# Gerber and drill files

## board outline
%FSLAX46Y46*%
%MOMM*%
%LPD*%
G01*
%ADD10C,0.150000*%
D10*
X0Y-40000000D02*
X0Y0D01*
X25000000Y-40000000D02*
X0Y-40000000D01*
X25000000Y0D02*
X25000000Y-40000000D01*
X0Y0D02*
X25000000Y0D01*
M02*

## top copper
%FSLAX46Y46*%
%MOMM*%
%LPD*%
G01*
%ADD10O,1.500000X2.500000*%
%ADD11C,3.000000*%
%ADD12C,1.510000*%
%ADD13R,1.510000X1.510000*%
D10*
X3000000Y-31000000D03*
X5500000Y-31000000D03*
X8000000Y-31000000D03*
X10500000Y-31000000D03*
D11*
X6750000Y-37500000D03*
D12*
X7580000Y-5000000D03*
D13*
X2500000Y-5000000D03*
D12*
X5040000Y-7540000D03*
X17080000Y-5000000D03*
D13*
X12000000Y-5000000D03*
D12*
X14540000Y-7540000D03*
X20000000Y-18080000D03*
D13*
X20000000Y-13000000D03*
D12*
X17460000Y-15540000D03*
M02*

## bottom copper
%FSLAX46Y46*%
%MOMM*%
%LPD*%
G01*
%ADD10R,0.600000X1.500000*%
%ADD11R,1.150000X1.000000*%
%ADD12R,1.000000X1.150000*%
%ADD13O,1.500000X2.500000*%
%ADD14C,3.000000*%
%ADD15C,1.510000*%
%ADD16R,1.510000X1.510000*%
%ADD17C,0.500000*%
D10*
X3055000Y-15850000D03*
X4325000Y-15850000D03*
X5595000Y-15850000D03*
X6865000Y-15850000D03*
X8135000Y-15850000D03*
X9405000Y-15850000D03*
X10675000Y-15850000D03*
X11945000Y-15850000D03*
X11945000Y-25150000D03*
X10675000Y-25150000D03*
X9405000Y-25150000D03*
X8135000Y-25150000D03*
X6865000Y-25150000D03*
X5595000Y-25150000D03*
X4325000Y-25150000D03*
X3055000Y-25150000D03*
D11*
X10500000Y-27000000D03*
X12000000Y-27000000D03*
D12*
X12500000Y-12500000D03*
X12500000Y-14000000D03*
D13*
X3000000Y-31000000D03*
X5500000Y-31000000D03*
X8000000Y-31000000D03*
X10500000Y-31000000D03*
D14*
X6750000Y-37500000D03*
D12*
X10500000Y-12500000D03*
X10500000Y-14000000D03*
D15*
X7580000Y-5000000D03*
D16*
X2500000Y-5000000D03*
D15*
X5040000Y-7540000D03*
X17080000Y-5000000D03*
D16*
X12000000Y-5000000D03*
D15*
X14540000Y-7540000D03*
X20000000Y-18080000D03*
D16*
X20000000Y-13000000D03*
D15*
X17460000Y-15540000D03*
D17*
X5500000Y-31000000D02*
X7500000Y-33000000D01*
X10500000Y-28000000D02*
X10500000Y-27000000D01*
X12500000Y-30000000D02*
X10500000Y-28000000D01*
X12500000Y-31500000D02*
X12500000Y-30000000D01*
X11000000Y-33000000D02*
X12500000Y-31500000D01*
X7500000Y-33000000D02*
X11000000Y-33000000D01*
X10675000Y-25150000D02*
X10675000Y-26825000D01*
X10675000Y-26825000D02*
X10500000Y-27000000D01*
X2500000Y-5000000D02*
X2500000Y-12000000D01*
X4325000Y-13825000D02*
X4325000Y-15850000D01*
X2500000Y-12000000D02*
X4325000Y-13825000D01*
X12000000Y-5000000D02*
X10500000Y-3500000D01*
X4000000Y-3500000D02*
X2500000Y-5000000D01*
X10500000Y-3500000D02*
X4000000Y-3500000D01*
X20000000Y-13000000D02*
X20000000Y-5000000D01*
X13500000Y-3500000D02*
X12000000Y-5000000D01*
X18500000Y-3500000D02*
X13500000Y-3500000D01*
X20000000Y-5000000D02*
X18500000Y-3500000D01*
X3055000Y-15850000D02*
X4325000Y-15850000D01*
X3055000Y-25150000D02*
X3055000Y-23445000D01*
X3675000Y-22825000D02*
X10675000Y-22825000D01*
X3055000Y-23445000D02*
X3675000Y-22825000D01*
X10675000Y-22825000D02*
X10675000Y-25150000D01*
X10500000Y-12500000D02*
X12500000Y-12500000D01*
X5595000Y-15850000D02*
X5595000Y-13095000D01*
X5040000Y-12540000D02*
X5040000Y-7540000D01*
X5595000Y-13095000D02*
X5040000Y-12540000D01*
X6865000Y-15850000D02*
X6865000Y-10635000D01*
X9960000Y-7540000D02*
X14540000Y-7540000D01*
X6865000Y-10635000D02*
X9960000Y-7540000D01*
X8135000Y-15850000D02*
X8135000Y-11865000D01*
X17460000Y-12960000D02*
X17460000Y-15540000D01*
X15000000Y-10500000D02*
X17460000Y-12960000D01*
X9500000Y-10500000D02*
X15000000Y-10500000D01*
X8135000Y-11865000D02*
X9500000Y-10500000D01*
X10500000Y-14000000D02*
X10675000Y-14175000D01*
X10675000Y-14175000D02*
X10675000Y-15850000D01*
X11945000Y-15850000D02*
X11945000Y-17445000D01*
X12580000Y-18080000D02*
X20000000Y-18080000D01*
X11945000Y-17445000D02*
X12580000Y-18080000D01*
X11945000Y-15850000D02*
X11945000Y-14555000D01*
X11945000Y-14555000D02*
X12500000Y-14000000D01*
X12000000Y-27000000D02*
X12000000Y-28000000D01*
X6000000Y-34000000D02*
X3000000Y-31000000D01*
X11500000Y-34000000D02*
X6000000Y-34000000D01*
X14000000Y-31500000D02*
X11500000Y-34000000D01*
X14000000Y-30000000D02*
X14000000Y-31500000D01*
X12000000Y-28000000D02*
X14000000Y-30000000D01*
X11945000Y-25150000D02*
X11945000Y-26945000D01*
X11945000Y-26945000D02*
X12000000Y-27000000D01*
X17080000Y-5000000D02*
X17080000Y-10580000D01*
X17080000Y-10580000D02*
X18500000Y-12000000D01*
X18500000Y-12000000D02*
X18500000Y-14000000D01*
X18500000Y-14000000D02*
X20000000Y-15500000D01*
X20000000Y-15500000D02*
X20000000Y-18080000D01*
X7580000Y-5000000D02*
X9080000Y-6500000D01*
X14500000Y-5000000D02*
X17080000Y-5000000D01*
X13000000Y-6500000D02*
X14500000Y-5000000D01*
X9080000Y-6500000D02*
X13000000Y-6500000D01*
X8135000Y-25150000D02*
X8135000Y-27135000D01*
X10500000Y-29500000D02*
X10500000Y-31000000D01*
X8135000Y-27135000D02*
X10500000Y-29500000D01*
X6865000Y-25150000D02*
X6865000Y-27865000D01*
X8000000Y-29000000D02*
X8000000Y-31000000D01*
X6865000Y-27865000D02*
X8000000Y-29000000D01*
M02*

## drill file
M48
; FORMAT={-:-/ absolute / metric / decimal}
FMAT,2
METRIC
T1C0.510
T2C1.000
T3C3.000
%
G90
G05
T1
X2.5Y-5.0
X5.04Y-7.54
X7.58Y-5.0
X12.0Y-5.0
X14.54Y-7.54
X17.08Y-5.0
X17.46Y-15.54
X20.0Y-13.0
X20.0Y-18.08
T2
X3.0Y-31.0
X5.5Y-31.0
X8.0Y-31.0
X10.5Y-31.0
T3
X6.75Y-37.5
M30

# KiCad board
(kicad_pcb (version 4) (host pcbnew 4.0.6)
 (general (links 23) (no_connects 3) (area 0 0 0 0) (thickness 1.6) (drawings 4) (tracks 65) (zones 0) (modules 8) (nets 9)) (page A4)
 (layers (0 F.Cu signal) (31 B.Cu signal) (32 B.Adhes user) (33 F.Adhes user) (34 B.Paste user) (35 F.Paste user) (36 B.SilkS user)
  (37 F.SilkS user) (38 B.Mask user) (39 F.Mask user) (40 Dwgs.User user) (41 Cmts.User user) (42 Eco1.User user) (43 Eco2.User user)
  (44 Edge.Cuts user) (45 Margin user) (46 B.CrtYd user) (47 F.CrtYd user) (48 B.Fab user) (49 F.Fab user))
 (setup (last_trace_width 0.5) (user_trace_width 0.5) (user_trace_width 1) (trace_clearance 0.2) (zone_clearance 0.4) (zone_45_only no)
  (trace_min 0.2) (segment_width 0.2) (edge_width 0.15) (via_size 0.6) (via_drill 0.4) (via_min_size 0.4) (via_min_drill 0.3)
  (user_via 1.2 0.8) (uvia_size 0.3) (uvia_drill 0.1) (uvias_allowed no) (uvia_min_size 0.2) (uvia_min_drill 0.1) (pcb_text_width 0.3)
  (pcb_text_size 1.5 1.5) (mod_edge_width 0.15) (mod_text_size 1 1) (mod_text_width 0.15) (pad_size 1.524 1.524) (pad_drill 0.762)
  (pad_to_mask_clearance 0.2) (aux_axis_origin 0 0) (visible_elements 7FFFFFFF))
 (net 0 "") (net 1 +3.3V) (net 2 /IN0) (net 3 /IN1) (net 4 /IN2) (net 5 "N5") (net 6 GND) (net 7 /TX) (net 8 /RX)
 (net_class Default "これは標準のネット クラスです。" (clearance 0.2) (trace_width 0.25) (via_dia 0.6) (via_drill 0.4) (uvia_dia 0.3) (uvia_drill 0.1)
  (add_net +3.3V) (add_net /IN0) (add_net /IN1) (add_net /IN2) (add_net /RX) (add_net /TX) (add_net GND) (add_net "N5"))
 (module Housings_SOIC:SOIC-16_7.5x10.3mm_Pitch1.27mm (layer B.Cu) (at 7.5 20.5 270)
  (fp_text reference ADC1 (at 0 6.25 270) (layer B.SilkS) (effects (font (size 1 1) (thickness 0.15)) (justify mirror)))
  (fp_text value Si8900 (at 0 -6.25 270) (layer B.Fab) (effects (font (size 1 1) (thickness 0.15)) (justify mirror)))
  (pad 1 smd rect (at -4.65 4.445 270) (size 1.5 0.6) (layers B.Cu B.Paste B.Mask) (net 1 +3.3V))
  (pad 2 smd rect (at -4.65 3.175 270) (size 1.5 0.6) (layers B.Cu B.Paste B.Mask) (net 1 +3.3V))
  (pad 3 smd rect (at -4.65 1.905 270) (size 1.5 0.6) (layers B.Cu B.Paste B.Mask) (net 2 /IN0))
  (pad 4 smd rect (at -4.65 0.635 270) (size 1.5 0.6) (layers B.Cu B.Paste B.Mask) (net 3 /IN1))
  (pad 5 smd rect (at -4.65 -0.635 270) (size 1.5 0.6) (layers B.Cu B.Paste B.Mask) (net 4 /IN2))
  (pad 6 smd rect (at -4.65 -1.905 270) (size 1.5 0.6) (layers B.Cu B.Paste B.Mask))
  (pad 7 smd rect (at -4.65 -3.175 270) (size 1.5 0.6) (layers B.Cu B.Paste B.Mask) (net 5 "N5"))
  (pad 8 smd rect (at -4.65 -4.445 270) (size 1.5 0.6) (layers B.Cu B.Paste B.Mask) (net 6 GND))
  (pad 9 smd rect (at 4.65 -4.445 270) (size 1.5 0.6) (layers B.Cu B.Paste B.Mask) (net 6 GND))
  (pad 10 smd rect (at 4.65 -3.175 270) (size 1.5 0.6) (layers B.Cu B.Paste B.Mask) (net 1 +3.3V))
  (pad 11 smd rect (at 4.65 -1.905 270) (size 1.5 0.6) (layers B.Cu B.Paste B.Mask))
  (pad 12 smd rect (at 4.65 -0.635 270) (size 1.5 0.6) (layers B.Cu B.Paste B.Mask) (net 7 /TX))
  (pad 13 smd rect (at 4.65 0.635 270) (size 1.5 0.6) (layers B.Cu B.Paste B.Mask) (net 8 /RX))
  (pad 14 smd rect (at 4.65 1.905 270) (size 1.5 0.6) (layers B.Cu B.Paste B.Mask))
  (pad 15 smd rect (at 4.65 3.175 270) (size 1.5 0.6) (layers B.Cu B.Paste B.Mask))
  (pad 16 smd rect (at 4.65 4.445 270) (size 1.5 0.6) (layers B.Cu B.Paste B.Mask) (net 1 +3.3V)))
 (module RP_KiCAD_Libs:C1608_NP (layer B.Cu) (at 11.5 27)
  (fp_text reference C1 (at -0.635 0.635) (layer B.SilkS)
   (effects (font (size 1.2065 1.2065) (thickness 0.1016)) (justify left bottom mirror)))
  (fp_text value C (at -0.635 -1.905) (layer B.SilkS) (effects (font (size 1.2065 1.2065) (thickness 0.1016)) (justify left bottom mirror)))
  (pad 1 smd rect (at -1 0) (size 1.15 1) (layers B.Cu B.Paste B.Mask) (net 1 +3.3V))
  (pad 2 smd rect (at 0.5 0) (size 1.15 1) (layers B.Cu B.Paste B.Mask) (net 6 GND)))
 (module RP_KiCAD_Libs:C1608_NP (layer B.Cu) (at 12.5 13.5 270)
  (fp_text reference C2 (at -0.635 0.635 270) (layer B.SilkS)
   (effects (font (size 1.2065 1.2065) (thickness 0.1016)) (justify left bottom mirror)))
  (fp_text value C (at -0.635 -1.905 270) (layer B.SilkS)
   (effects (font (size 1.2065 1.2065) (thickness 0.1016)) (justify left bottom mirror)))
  (pad 1 smd rect (at -1 0 270) (size 1.15 1) (layers B.Cu B.Paste B.Mask) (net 1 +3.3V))
  (pad 2 smd rect (at 0.5 0 270) (size 1.15 1) (layers B.Cu B.Paste B.Mask) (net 6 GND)))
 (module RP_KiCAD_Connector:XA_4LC (layer F.Cu) (at 3 31)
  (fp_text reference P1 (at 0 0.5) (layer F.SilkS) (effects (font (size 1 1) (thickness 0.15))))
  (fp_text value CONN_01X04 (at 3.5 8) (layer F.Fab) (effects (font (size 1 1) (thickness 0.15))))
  (pad 1 thru_hole oval (at 0 0) (size 1.5 2.5) (drill 1) (layers *.Cu *.Mask F.SilkS) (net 6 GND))
  (pad 2 thru_hole oval (at 2.5 0) (size 1.5 2.5) (drill 1) (layers *.Cu *.Mask F.SilkS) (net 1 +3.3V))
  (pad 3 thru_hole oval (at 5 0) (size 1.5 2.5) (drill 1) (layers *.Cu *.Mask F.SilkS) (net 8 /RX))
  (pad 4 thru_hole oval (at 7.5 0) (size 1.5 2.5) (drill 1) (layers *.Cu *.Mask F.SilkS) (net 7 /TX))
  (pad "" thru_hole circle (at 3.75 6.5) (size 3 3) (drill 3) (layers *.Cu *.Mask F.SilkS) (clearance -0.3)))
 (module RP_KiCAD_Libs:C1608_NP (layer B.Cu) (at 10.5 13.5 270)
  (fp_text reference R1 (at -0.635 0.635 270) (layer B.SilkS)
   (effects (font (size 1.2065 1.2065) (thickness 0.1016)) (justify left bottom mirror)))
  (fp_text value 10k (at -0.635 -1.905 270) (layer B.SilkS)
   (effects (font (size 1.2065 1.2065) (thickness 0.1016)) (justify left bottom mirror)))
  (pad 1 smd rect (at -1 0 270) (size 1.15 1) (layers B.Cu B.Paste B.Mask) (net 1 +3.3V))
  (pad 2 smd rect (at 0.5 0 270) (size 1.15 1) (layers B.Cu B.Paste B.Mask) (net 5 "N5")))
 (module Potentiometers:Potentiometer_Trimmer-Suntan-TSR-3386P (layer F.Cu) (at 2.5 5)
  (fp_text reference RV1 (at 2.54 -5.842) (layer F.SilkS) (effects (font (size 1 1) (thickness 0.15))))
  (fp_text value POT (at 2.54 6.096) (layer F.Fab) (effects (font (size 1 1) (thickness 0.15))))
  (pad 3 thru_hole circle (at 5.08 0) (size 1.51 1.51) (drill 0.51) (layers *.Cu *.Mask F.SilkS) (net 6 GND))
  (pad 1 thru_hole rect (at 0 0) (size 1.51 1.51) (drill 0.51) (layers *.Cu *.Mask F.SilkS) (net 1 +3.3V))
  (pad 2 thru_hole circle (at 2.54 2.54) (size 1.51 1.51) (drill 0.51) (layers *.Cu *.Mask F.SilkS) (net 2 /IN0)))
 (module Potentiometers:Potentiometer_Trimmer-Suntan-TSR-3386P (layer F.Cu) (at 12 5)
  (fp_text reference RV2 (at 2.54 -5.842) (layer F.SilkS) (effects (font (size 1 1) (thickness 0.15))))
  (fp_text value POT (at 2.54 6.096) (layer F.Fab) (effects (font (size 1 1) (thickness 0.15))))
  (pad 3 thru_hole circle (at 5.08 0) (size 1.51 1.51) (drill 0.51) (layers *.Cu *.Mask F.SilkS) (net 6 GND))
  (pad 1 thru_hole rect (at 0 0) (size 1.51 1.51) (drill 0.51) (layers *.Cu *.Mask F.SilkS) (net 1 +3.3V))
  (pad 2 thru_hole circle (at 2.54 2.54) (size 1.51 1.51) (drill 0.51) (layers *.Cu *.Mask F.SilkS) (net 3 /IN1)))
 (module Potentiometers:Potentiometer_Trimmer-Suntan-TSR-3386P (layer F.Cu) (at 20 13 270)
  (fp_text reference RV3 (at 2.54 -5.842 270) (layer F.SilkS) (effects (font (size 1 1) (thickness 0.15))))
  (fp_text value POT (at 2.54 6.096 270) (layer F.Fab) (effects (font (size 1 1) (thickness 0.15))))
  (pad 3 thru_hole circle (at 5.08 0 270) (size 1.51 1.51) (drill 0.51) (layers *.Cu *.Mask F.SilkS) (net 6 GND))
  (pad 1 thru_hole rect (at 0 0 270) (size 1.51 1.51) (drill 0.51) (layers *.Cu *.Mask F.SilkS) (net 1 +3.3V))
  (pad 2 thru_hole circle (at 2.54 2.54 270) (size 1.51 1.51) (drill 0.51) (layers *.Cu *.Mask F.SilkS) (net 4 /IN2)))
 (gr_line (start 0 40) (end 0 0) (angle 90) (layer Edge.Cuts) (width 0.15))
 (gr_line (start 25 40) (end 0 40) (angle 90) (layer Edge.Cuts) (width 0.15))
 (gr_line (start 25 0) (end 25 40) (angle 90) (layer Edge.Cuts) (width 0.15))
 (gr_line (start 0 0) (end 25 0) (angle 90) (layer Edge.Cuts) (width 0.15))
 (segment (start 5.5 31) (end 7.5 33) (width 0.5) (layer B.Cu) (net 1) (status 400000))
 (segment (start 10.5 28) (end 10.5 27) (width 0.5) (layer B.Cu) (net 1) (status 800000))
 (segment (start 12.5 30) (end 10.5 28) (width 0.5) (layer B.Cu) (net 1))
 (segment (start 12.5 31.5) (end 12.5 30) (width 0.5) (layer B.Cu) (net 1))
 (segment (start 11 33) (end 12.5 31.5) (width 0.5) (layer B.Cu) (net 1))
 (segment (start 7.5 33) (end 11 33) (width 0.5) (layer B.Cu) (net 1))
 (segment (start 10.675 25.15) (end 10.675 26.825) (width 0.5) (layer B.Cu) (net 1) (status C00000))
 (segment (start 10.675 26.825) (end 10.5 27) (width 0.5) (layer B.Cu) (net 1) (status C00000))
 (segment (start 2.5 5) (end 2.5 12) (width 0.5) (layer B.Cu) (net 1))
 (segment (start 4.325 13.825) (end 4.325 15.85) (width 0.5) (layer B.Cu) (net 1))
 (segment (start 2.5 12) (end 4.325 13.825) (width 0.5) (layer B.Cu) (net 1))
 (segment (start 12 5) (end 10.5 3.5) (width 0.5) (layer B.Cu) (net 1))
 (segment (start 4 3.5) (end 2.5 5) (width 0.5) (layer B.Cu) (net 1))
 (segment (start 10.5 3.5) (end 4 3.5) (width 0.5) (layer B.Cu) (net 1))
 (segment (start 20 13) (end 20 5) (width 0.5) (layer B.Cu) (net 1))
 (segment (start 13.5 3.5) (end 12 5) (width 0.5) (layer B.Cu) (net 1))
 (segment (start 18.5 3.5) (end 13.5 3.5) (width 0.5) (layer B.Cu) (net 1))
 (segment (start 20 5) (end 18.5 3.5) (width 0.5) (layer B.Cu) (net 1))
 (segment (start 3.055 15.85) (end 4.325 15.85) (width 0.5) (layer B.Cu) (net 1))
 (segment (start 3.055 25.15) (end 3.055 23.445) (width 0.5) (layer B.Cu) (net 1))
 (segment (start 3.675 22.825) (end 10.675 22.825) (width 0.5) (layer B.Cu) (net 1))
 (segment (start 3.055 23.445) (end 3.675 22.825) (width 0.5) (layer B.Cu) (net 1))
 (segment (start 10.675 22.825) (end 10.675 25.15) (width 0.5) (layer B.Cu) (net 1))
 (segment (start 10.5 12.5) (end 12.5 12.5) (width 0.5) (layer B.Cu) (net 1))
 (segment (start 5.595 15.85) (end 5.595 13.095) (width 0.5) (layer B.Cu) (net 2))
 (segment (start 5.04 12.54) (end 5.04 7.54) (width 0.5) (layer B.Cu) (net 2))
 (segment (start 5.595 13.095) (end 5.04 12.54) (width 0.5) (layer B.Cu) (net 2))
 (segment (start 6.865 15.85) (end 6.865 10.635) (width 0.5) (layer B.Cu) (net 3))
 (segment (start 9.96 7.54) (end 14.54 7.54) (width 0.5) (layer B.Cu) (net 3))
 (segment (start 6.865 10.635) (end 9.96 7.54) (width 0.5) (layer B.Cu) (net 3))
 (segment (start 8.135 15.85) (end 8.135 11.865) (width 0.5) (layer B.Cu) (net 4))
 (segment (start 17.46 12.96) (end 17.46 15.54) (width 0.5) (layer B.Cu) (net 4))
 (segment (start 15 10.5) (end 17.46 12.96) (width 0.5) (layer B.Cu) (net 4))
 (segment (start 9.5 10.5) (end 15 10.5) (width 0.5) (layer B.Cu) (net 4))
 (segment (start 8.135 11.865) (end 9.5 10.5) (width 0.5) (layer B.Cu) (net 4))
 (segment (start 10.5 14) (end 10.675 14.175) (width 0.5) (layer B.Cu) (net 5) (status C00000))
 (segment (start 10.675 14.175) (end 10.675 15.85) (width 0.5) (layer B.Cu) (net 5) (status C00000))
 (segment (start 11.945 15.85) (end 11.945 17.445) (width 0.5) (layer B.Cu) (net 6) (status 400000))
 (segment (start 12.58 18.08) (end 20 18.08) (width 0.5) (layer B.Cu) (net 6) (status 800000))
 (segment (start 11.945 17.445) (end 12.58 18.08) (width 0.5) (layer B.Cu) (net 6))
 (segment (start 11.945 15.85) (end 11.945 14.555) (width 0.5) (layer B.Cu) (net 6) (status 400000))
 (segment (start 11.945 14.555) (end 12.5 14) (width 0.5) (layer B.Cu) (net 6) (status 800000))
 (segment (start 12 27) (end 12 28) (width 0.5) (layer B.Cu) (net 6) (status 400000))
 (segment (start 6 34) (end 3 31) (width 0.5) (layer B.Cu) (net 6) (status 800000))
 (segment (start 11.5 34) (end 6 34) (width 0.5) (layer B.Cu) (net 6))
 (segment (start 14 31.5) (end 11.5 34) (width 0.5) (layer B.Cu) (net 6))
 (segment (start 14 30) (end 14 31.5) (width 0.5) (layer B.Cu) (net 6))
 (segment (start 12 28) (end 14 30) (width 0.5) (layer B.Cu) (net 6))
 (segment (start 11.945 25.15) (end 11.945 26.945) (width 0.5) (layer B.Cu) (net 6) (status C00000))
 (segment (start 11.945 26.945) (end 12 27) (width 0.5) (layer B.Cu) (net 6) (status C00000))
 (segment (start 17.08 5) (end 17.08 10.58) (width 0.5) (layer B.Cu) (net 6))
 (segment (start 17.08 10.58) (end 18.5 12) (width 0.5) (layer B.Cu) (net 6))
 (segment (start 18.5 12) (end 18.5 14) (width 0.5) (layer B.Cu) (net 6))
 (segment (start 18.5 14) (end 20 15.5) (width 0.5) (layer B.Cu) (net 6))
 (segment (start 20 15.5) (end 20 18.08) (width 0.5) (layer B.Cu) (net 6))
 (segment (start 7.58 5) (end 9.08 6.5) (width 0.5) (layer B.Cu) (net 6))
 (segment (start 14.5 5) (end 17.08 5) (width 0.5) (layer B.Cu) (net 6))
 (segment (start 13 6.5) (end 14.5 5) (width 0.5) (layer B.Cu) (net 6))
 (segment (start 9.08 6.5) (end 13 6.5) (width 0.5) (layer B.Cu) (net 6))
 (segment (start 8.135 25.15) (end 8.135 27.135) (width 0.5) (layer B.Cu) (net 7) (status 400000))
 (segment (start 10.5 29.5) (end 10.5 31) (width 0.5) (layer B.Cu) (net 7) (status 800000))
 (segment (start 8.135 27.135) (end 10.5 29.5) (width 0.5) (layer B.Cu) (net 7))
 (segment (start 6.865 25.15) (end 6.865 27.865) (width 0.5) (layer B.Cu) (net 8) (status 400000))
 (segment (start 8 29) (end 8 31) (width 0.5) (layer B.Cu) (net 8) (status 800000))
 (segment (start 6.865 27.865) (end 8 29) (width 0.5) (layer B.Cu) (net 8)))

